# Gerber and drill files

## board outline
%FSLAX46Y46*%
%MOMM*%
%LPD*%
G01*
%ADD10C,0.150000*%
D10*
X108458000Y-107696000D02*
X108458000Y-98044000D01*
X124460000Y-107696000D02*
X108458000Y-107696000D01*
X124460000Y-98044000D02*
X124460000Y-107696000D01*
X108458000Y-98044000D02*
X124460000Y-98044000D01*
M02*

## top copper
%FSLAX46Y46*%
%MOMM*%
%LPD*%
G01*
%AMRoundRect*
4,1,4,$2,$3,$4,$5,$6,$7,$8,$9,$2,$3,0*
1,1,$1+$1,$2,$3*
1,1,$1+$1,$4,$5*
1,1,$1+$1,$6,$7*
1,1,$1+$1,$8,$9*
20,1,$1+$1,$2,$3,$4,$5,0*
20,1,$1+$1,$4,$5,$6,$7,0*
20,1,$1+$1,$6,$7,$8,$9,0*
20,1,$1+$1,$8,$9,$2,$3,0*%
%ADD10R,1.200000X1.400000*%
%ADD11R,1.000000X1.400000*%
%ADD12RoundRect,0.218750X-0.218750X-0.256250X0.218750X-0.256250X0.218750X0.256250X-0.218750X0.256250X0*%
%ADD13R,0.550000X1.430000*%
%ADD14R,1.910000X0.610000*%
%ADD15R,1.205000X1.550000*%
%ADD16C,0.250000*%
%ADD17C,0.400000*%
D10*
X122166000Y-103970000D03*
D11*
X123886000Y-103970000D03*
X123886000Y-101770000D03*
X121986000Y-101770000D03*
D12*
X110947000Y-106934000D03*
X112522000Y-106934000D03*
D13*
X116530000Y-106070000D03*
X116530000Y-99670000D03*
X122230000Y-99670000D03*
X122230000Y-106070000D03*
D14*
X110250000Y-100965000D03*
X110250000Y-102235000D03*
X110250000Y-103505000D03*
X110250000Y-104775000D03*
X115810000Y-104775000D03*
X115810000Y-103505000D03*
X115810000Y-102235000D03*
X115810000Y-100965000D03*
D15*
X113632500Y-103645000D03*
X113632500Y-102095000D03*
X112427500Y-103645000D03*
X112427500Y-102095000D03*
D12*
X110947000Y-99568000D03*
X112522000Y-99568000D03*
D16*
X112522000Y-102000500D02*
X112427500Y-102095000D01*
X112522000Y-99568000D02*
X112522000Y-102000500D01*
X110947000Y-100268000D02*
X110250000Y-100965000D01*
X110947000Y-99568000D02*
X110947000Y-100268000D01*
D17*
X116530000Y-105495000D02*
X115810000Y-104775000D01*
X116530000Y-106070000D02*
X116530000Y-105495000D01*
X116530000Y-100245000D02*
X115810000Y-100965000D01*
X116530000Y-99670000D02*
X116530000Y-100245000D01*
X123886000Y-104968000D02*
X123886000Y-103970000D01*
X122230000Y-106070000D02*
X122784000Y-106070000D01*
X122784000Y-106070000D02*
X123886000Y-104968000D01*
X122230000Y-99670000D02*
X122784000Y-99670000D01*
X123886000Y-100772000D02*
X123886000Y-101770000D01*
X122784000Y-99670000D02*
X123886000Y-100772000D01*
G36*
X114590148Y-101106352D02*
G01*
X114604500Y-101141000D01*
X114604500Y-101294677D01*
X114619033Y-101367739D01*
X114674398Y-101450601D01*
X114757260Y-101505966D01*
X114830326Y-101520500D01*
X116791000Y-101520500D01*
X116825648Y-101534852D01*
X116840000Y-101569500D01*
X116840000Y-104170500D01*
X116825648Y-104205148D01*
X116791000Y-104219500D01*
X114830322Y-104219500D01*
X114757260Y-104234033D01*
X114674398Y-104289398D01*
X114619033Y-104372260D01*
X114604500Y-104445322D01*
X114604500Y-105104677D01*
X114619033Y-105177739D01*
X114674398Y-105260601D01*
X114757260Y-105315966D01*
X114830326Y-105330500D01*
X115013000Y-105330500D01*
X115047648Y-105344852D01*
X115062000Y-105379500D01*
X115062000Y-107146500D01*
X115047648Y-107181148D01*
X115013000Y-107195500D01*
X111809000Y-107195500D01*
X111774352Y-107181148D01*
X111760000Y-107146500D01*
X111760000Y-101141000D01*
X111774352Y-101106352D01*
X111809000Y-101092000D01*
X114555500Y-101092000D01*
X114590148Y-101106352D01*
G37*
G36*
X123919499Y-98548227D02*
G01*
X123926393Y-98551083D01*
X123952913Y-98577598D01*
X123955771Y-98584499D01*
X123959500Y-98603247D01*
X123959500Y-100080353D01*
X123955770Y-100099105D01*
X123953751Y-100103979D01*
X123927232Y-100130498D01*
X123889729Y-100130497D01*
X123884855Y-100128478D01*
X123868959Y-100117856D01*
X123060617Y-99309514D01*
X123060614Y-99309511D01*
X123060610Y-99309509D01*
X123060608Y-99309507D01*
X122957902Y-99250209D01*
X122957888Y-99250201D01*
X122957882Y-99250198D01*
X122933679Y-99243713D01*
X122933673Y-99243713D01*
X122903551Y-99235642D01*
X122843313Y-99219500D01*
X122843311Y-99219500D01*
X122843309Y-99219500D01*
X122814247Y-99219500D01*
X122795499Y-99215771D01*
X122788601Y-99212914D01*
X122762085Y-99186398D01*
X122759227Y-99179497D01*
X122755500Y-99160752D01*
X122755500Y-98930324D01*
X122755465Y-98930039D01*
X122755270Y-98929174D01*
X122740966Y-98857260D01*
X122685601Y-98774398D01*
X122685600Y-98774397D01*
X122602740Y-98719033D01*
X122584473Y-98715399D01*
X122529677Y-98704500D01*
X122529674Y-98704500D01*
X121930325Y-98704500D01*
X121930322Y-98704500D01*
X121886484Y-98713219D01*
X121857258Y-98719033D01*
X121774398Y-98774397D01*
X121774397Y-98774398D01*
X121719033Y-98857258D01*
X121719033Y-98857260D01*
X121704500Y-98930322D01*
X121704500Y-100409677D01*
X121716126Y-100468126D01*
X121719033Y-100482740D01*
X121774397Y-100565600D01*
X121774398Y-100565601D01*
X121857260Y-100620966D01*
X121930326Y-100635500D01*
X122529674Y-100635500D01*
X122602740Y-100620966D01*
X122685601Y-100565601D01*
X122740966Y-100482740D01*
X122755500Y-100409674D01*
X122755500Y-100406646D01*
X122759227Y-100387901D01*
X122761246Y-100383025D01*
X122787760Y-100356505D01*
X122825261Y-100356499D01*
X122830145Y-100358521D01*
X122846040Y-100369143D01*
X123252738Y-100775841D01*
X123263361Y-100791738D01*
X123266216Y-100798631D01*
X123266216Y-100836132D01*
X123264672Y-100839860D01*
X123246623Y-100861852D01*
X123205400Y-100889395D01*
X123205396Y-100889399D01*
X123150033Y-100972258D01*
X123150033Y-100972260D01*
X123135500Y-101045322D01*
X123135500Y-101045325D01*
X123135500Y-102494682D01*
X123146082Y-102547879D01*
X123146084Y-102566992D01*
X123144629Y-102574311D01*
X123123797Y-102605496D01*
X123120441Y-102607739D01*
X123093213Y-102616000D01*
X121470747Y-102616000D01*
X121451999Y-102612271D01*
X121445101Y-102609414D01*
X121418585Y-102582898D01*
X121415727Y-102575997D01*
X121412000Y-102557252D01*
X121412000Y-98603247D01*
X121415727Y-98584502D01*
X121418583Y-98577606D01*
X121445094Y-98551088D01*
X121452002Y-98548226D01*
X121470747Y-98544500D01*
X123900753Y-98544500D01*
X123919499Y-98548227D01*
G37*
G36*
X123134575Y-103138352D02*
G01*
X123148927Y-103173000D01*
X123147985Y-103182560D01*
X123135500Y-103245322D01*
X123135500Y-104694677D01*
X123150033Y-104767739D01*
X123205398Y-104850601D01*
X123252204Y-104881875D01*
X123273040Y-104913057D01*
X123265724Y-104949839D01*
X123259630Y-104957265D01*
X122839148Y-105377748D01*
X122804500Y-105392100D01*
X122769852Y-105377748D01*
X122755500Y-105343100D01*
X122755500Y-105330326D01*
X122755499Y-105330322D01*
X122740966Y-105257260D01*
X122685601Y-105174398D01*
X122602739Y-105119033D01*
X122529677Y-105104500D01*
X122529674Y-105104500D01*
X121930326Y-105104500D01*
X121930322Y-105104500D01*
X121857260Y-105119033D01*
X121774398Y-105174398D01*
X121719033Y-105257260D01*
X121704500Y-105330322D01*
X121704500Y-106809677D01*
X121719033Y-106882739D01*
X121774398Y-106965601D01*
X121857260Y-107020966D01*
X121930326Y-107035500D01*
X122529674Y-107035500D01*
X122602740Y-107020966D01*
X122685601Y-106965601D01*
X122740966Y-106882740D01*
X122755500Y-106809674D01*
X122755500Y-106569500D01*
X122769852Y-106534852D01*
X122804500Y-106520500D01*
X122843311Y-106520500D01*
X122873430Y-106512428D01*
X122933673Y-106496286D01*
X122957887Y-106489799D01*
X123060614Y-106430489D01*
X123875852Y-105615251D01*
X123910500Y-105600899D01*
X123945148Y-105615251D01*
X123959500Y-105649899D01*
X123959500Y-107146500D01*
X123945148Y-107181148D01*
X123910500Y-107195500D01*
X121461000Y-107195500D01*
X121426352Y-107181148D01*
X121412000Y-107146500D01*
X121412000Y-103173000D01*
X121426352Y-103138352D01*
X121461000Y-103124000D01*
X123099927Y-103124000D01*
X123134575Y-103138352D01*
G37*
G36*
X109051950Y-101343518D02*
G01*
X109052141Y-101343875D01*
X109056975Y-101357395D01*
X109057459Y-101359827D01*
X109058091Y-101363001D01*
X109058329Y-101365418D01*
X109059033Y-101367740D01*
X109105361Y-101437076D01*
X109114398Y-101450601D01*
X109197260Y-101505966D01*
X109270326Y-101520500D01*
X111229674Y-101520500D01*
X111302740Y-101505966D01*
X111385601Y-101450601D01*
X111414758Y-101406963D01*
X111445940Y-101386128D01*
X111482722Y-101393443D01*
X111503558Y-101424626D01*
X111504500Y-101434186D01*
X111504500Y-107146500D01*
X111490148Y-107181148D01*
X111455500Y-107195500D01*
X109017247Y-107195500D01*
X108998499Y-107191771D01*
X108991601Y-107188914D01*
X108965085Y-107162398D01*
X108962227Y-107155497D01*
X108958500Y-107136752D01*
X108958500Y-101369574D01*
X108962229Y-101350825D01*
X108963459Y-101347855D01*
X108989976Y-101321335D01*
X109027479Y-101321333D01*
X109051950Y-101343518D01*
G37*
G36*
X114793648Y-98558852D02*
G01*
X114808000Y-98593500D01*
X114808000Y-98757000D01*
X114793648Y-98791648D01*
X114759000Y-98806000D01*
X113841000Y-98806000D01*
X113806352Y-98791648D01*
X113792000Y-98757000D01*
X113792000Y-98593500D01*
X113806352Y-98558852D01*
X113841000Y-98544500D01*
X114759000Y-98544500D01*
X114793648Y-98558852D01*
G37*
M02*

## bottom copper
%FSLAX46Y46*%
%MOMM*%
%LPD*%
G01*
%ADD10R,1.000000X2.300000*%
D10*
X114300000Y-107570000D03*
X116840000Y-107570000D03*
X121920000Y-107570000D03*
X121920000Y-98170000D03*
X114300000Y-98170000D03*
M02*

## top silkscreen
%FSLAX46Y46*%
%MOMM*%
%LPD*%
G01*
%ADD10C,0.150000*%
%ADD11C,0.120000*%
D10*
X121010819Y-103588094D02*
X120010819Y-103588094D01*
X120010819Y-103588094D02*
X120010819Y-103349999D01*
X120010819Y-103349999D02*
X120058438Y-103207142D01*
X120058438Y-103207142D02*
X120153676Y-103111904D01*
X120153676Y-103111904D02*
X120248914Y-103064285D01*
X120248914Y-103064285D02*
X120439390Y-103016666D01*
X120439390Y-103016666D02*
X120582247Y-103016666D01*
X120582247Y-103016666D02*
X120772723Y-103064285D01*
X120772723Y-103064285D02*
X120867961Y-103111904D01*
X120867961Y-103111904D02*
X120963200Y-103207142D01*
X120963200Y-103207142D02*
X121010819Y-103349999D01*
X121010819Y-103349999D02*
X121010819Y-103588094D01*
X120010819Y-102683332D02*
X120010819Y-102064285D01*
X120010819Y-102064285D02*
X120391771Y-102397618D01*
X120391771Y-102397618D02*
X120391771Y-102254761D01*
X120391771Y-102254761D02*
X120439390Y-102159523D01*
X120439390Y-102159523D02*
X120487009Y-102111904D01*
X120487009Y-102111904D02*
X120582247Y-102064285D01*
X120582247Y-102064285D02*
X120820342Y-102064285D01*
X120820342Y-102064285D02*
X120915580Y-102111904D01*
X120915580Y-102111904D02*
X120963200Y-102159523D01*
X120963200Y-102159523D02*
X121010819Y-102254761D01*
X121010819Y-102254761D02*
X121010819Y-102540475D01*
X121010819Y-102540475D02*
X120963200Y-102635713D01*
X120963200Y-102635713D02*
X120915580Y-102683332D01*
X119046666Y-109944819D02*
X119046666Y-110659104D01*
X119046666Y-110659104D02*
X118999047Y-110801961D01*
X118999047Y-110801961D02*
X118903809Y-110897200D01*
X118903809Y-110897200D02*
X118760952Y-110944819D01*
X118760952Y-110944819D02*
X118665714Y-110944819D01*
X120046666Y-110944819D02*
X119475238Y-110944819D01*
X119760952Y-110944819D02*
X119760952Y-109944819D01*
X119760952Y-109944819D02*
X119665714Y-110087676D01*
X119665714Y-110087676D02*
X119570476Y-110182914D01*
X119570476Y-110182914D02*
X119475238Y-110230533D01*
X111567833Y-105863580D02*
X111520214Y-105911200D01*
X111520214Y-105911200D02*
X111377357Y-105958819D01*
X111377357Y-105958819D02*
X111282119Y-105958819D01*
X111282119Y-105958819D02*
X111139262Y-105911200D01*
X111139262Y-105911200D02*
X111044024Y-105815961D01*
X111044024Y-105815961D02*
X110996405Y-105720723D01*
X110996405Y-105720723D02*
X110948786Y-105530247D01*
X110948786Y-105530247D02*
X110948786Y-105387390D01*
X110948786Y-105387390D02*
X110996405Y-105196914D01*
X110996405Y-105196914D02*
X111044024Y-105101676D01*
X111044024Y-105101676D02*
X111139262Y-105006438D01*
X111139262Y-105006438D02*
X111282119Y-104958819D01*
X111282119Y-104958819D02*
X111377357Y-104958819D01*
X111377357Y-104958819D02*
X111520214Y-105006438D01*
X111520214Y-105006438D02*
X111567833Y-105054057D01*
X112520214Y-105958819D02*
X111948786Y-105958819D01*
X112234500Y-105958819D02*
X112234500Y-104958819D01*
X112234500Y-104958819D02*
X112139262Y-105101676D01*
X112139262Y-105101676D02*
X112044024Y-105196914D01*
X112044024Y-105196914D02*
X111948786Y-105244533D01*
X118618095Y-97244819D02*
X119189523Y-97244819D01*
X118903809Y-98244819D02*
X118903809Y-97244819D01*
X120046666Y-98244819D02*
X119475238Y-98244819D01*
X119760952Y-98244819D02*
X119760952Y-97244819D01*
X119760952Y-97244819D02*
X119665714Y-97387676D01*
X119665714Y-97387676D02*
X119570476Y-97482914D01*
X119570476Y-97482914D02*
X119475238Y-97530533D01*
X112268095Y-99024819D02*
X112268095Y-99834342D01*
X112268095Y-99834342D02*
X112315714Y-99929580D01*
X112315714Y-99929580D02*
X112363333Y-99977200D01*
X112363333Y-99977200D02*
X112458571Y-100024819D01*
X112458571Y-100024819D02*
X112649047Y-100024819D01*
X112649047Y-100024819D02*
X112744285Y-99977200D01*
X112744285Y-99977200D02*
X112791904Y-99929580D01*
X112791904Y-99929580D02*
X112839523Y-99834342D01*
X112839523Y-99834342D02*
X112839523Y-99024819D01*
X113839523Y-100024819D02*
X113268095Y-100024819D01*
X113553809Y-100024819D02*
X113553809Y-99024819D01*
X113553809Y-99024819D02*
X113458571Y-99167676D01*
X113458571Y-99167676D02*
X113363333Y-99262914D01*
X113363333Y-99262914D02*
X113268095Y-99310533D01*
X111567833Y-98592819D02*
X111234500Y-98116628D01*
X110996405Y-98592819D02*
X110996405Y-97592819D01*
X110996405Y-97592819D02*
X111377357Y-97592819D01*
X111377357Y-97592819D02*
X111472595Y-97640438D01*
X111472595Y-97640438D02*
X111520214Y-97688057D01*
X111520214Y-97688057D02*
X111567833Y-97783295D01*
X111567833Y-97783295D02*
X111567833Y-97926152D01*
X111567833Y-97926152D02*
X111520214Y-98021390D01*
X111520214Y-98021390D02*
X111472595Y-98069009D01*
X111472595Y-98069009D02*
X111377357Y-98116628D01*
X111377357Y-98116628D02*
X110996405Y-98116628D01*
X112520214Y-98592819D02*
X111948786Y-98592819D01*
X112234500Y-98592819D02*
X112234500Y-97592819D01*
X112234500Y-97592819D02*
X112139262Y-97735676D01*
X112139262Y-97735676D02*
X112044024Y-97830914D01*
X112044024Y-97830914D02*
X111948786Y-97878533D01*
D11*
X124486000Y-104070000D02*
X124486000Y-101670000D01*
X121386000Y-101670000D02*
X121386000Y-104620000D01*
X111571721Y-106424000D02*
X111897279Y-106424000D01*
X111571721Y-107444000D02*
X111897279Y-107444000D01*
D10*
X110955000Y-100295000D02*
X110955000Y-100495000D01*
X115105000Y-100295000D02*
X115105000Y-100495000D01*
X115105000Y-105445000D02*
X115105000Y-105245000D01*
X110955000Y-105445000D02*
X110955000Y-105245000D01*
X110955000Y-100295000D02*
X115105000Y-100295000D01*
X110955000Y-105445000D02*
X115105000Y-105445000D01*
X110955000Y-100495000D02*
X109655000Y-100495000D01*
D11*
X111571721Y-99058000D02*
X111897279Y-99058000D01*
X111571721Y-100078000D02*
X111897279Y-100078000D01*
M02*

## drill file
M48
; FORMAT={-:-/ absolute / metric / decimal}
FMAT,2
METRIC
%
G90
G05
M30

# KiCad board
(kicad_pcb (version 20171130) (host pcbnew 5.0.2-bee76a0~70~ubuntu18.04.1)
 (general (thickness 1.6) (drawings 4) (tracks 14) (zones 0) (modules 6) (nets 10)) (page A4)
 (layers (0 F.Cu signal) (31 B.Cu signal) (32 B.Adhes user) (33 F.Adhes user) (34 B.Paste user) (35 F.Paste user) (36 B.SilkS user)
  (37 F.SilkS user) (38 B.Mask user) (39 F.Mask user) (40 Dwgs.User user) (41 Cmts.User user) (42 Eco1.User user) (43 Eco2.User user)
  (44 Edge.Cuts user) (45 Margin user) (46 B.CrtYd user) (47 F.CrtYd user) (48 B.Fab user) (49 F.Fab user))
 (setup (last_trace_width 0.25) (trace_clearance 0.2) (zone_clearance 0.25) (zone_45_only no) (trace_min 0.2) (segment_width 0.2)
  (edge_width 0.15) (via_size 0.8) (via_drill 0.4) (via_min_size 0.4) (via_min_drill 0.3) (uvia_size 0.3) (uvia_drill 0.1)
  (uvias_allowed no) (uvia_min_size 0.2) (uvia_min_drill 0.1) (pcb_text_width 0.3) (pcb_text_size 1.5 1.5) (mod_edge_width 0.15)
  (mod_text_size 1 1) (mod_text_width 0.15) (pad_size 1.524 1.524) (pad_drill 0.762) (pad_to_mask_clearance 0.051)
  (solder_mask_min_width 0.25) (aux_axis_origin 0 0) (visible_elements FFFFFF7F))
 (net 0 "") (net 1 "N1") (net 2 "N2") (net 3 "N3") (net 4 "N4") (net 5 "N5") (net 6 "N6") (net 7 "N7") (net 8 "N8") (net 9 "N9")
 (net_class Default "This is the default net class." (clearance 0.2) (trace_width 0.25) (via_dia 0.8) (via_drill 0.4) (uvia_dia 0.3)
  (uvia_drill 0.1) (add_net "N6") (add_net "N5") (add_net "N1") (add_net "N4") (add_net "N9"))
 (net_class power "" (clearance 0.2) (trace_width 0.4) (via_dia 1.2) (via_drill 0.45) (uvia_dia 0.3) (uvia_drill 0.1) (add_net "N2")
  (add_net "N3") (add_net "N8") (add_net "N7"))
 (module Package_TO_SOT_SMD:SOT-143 (layer F.Cu) (at 122.936 102.87 90)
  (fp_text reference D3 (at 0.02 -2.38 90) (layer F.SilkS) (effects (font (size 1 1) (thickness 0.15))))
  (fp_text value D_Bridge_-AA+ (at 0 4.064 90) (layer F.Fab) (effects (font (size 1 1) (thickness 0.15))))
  (fp_line (start -1.2 1.55) (end 1.2 1.55) (layer F.SilkS) (width 0.12))
  (fp_line (start 1.2 -1.55) (end -1.75 -1.55) (layer F.SilkS) (width 0.12))
  (pad 1 smd rect (at -1.1 -0.77) (size 1.2 1.4) (layers F.Cu F.Paste F.Mask) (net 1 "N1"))
  (pad 2 smd rect (at -1.1 0.95) (size 1 1.4) (layers F.Cu F.Paste F.Mask) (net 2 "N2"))
  (pad 3 smd rect (at 1.1 0.95) (size 1 1.4) (layers F.Cu F.Paste F.Mask) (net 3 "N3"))
  (pad 4 smd rect (at 1.1 -0.95) (size 1 1.4) (layers F.Cu F.Paste F.Mask) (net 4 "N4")))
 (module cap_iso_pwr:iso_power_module (layer F.Cu) (at 119.38 102.87)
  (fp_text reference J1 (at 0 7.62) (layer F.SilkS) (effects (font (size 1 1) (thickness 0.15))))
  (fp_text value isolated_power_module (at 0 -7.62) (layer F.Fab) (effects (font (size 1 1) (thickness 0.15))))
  (pad 1 smd rect (at -5.08 4.7) (size 1 2.3) (layers B.Cu B.Paste B.Mask) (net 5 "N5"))
  (pad 3 smd rect (at -2.54 4.7) (size 1 2.3) (layers B.Cu B.Paste B.Mask) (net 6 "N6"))
  (pad 7 smd rect (at 2.54 4.7) (size 1 2.3) (layers B.Cu B.Paste B.Mask) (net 1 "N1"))
  (pad 8 smd rect (at 2.54 -4.7) (size 1 2.3) (layers B.Cu B.Paste B.Mask) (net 4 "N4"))
  (pad 14 smd rect (at -5.08 -4.7) (size 1 2.3) (layers B.Cu B.Paste B.Mask)))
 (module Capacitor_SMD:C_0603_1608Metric (layer F.Cu) (at 111.7345 106.934)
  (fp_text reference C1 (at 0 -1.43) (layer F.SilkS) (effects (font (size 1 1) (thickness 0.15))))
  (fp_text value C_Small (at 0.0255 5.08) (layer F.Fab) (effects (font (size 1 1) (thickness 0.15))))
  (fp_line (start -0.162779 -0.51) (end 0.162779 -0.51) (layer F.SilkS) (width 0.12))
  (fp_line (start -0.162779 0.51) (end 0.162779 0.51) (layer F.SilkS) (width 0.12))
  (pad 1 smd roundrect (at -0.7875 0) (size 0.875 0.95) (layers F.Cu F.Paste F.Mask) (roundrect_rratio 0.25) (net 6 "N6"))
  (pad 2 smd roundrect (at 0.7875 0) (size 0.875 0.95) (layers F.Cu F.Paste F.Mask) (roundrect_rratio 0.25) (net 5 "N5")))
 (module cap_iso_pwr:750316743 (layer F.Cu) (at 119.38 102.87)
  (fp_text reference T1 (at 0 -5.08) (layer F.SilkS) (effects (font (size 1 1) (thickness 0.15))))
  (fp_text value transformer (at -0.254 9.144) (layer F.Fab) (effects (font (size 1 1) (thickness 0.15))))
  (pad 8 smd rect (at -2.85 3.2 90) (size 1.43 0.55) (layers F.Cu F.Paste F.Mask) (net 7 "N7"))
  (pad 1 smd rect (at -2.85 -3.2 90) (size 1.43 0.55) (layers F.Cu F.Paste F.Mask) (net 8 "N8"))
  (pad 4 smd rect (at 2.85 -3.2 90) (size 1.43 0.55) (layers F.Cu F.Paste F.Mask) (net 3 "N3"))
  (pad 5 smd rect (at 2.85 3.2 90) (size 1.43 0.55) (layers F.Cu F.Paste F.Mask) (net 2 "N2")))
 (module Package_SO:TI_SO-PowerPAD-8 (layer F.Cu) (at 113.03 102.87)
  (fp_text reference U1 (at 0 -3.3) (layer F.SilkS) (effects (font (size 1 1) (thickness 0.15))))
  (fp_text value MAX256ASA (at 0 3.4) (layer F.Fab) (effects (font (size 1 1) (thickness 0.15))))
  (fp_line (start -2.075 -2.575) (end -2.075 -2.375) (layer F.SilkS) (width 0.15))
  (fp_line (start 2.075 -2.575) (end 2.075 -2.375) (layer F.SilkS) (width 0.15))
  (fp_line (start 2.075 2.575) (end 2.075 2.375) (layer F.SilkS) (width 0.15))
  (fp_line (start -2.075 2.575) (end -2.075 2.375) (layer F.SilkS) (width 0.15))
  (fp_line (start -2.075 -2.575) (end 2.075 -2.575) (layer F.SilkS) (width 0.15))
  (fp_line (start -2.075 2.575) (end 2.075 2.575) (layer F.SilkS) (width 0.15))
  (fp_line (start -2.075 -2.375) (end -3.375 -2.375) (layer F.SilkS) (width 0.15))
  (pad 1 smd rect (at -2.78 -1.905) (size 1.91 0.61) (layers F.Cu F.Paste F.Mask) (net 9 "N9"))
  (pad 2 smd rect (at -2.78 -0.635) (size 1.91 0.61) (layers F.Cu F.Paste F.Mask) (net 6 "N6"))
  (pad 3 smd rect (at -2.78 0.635) (size 1.91 0.61) (layers F.Cu F.Paste F.Mask) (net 6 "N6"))
  (pad 4 smd rect (at -2.78 1.905) (size 1.91 0.61) (layers F.Cu F.Paste F.Mask) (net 6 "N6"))
  (pad 5 smd rect (at 2.78 1.905) (size 1.91 0.61) (layers F.Cu F.Paste F.Mask) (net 7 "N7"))
  (pad 6 smd rect (at 2.78 0.635) (size 1.91 0.61) (layers F.Cu F.Paste F.Mask) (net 5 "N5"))
  (pad 7 smd rect (at 2.78 -0.635) (size 1.91 0.61) (layers F.Cu F.Paste F.Mask) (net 5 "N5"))
  (pad 8 smd rect (at 2.78 -1.905) (size 1.91 0.61) (layers F.Cu F.Paste F.Mask) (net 8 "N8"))
  (pad 9 smd rect (at 0.6025 0.775) (size 1.205 1.55) (layers F.Cu F.Paste F.Mask) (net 5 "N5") (solder_paste_margin_ratio -0.2))
  (pad 9 smd rect (at 0.6025 -0.775) (size 1.205 1.55) (layers F.Cu F.Paste F.Mask) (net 5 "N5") (solder_paste_margin_ratio -0.2))
  (pad 9 smd rect (at -0.6025 0.775) (size 1.205 1.55) (layers F.Cu F.Paste F.Mask) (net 5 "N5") (solder_paste_margin_ratio -0.2))
  (pad 9 smd rect (at -0.6025 -0.775) (size 1.205 1.55) (layers F.Cu F.Paste F.Mask) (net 5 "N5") (solder_paste_margin_ratio -0.2)))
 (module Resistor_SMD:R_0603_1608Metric (layer F.Cu) (at 111.7345 99.568)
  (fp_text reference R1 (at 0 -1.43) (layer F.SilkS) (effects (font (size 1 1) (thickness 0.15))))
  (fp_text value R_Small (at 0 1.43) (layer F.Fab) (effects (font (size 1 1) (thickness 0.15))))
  (fp_line (start -0.162779 -0.51) (end 0.162779 -0.51) (layer F.SilkS) (width 0.12))
  (fp_line (start -0.162779 0.51) (end 0.162779 0.51) (layer F.SilkS) (width 0.12))
  (pad 1 smd roundrect (at -0.7875 0) (size 0.875 0.95) (layers F.Cu F.Paste F.Mask) (roundrect_rratio 0.25) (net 9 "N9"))
  (pad 2 smd roundrect (at 0.7875 0) (size 0.875 0.95) (layers F.Cu F.Paste F.Mask) (roundrect_rratio 0.25) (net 5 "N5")))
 (gr_line (start 108.458 107.696) (end 108.458 98.044) (layer Edge.Cuts) (width 0.15))
 (gr_line (start 124.46 107.696) (end 108.458 107.696) (layer Edge.Cuts) (width 0.15))
 (gr_line (start 124.46 98.044) (end 124.46 107.696) (layer Edge.Cuts) (width 0.15))
 (gr_line (start 108.458 98.044) (end 124.46 98.044) (layer Edge.Cuts) (width 0.15))
 (segment (start 112.522 102.0005) (end 112.4275 102.095) (width 0.25) (layer F.Cu) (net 5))
 (segment (start 112.522 99.568) (end 112.522 102.0005) (width 0.25) (layer F.Cu) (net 5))
 (segment (start 110.947 100.268) (end 110.25 100.965) (width 0.25) (layer F.Cu) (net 9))
 (segment (start 110.947 99.568) (end 110.947 100.268) (width 0.25) (layer F.Cu) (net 9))
 (segment (start 116.53 105.495) (end 115.81 104.775) (width 0.4) (layer F.Cu) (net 7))
 (segment (start 116.53 106.07) (end 116.53 105.495) (width 0.4) (layer F.Cu) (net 7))
 (segment (start 116.53 100.245) (end 115.81 100.965) (width 0.4) (layer F.Cu) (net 8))
 (segment (start 116.53 99.67) (end 116.53 100.245) (width 0.4) (layer F.Cu) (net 8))
 (segment (start 123.886 104.968) (end 123.886 103.97) (width 0.4) (layer F.Cu) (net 2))
 (segment (start 122.23 106.07) (end 122.784 106.07) (width 0.4) (layer F.Cu) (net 2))
 (segment (start 122.784 106.07) (end 123.886 104.968) (width 0.4) (layer F.Cu) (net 2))
 (segment (start 122.23 99.67) (end 122.784 99.67) (width 0.4) (layer F.Cu) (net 3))
 (segment (start 123.886 100.772) (end 123.886 101.77) (width 0.4) (layer F.Cu) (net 3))
 (segment (start 122.784 99.67) (end 123.886 100.772) (width 0.4) (layer F.Cu) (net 3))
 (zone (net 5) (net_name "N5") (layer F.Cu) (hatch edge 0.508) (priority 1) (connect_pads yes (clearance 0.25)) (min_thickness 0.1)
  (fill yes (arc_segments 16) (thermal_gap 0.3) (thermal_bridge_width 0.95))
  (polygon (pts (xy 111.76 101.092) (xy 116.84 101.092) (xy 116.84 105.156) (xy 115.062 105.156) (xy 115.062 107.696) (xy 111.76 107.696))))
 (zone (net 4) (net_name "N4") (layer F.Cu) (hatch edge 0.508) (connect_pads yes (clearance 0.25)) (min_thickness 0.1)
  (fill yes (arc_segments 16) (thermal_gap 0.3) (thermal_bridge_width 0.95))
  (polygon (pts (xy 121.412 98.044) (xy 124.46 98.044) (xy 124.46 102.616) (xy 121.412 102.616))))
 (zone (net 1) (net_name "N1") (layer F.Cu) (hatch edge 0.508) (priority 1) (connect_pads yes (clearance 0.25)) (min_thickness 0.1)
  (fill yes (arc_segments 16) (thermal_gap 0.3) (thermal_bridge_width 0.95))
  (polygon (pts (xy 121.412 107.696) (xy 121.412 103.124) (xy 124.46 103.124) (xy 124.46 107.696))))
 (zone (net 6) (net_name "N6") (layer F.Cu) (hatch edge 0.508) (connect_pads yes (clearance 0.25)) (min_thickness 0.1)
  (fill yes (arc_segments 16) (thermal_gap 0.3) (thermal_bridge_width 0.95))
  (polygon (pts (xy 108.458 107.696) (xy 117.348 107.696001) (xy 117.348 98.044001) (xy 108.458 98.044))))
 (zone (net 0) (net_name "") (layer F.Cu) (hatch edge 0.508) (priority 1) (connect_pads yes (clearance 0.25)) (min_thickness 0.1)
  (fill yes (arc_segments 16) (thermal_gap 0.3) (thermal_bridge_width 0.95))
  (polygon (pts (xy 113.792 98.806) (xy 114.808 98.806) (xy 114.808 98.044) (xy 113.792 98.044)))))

